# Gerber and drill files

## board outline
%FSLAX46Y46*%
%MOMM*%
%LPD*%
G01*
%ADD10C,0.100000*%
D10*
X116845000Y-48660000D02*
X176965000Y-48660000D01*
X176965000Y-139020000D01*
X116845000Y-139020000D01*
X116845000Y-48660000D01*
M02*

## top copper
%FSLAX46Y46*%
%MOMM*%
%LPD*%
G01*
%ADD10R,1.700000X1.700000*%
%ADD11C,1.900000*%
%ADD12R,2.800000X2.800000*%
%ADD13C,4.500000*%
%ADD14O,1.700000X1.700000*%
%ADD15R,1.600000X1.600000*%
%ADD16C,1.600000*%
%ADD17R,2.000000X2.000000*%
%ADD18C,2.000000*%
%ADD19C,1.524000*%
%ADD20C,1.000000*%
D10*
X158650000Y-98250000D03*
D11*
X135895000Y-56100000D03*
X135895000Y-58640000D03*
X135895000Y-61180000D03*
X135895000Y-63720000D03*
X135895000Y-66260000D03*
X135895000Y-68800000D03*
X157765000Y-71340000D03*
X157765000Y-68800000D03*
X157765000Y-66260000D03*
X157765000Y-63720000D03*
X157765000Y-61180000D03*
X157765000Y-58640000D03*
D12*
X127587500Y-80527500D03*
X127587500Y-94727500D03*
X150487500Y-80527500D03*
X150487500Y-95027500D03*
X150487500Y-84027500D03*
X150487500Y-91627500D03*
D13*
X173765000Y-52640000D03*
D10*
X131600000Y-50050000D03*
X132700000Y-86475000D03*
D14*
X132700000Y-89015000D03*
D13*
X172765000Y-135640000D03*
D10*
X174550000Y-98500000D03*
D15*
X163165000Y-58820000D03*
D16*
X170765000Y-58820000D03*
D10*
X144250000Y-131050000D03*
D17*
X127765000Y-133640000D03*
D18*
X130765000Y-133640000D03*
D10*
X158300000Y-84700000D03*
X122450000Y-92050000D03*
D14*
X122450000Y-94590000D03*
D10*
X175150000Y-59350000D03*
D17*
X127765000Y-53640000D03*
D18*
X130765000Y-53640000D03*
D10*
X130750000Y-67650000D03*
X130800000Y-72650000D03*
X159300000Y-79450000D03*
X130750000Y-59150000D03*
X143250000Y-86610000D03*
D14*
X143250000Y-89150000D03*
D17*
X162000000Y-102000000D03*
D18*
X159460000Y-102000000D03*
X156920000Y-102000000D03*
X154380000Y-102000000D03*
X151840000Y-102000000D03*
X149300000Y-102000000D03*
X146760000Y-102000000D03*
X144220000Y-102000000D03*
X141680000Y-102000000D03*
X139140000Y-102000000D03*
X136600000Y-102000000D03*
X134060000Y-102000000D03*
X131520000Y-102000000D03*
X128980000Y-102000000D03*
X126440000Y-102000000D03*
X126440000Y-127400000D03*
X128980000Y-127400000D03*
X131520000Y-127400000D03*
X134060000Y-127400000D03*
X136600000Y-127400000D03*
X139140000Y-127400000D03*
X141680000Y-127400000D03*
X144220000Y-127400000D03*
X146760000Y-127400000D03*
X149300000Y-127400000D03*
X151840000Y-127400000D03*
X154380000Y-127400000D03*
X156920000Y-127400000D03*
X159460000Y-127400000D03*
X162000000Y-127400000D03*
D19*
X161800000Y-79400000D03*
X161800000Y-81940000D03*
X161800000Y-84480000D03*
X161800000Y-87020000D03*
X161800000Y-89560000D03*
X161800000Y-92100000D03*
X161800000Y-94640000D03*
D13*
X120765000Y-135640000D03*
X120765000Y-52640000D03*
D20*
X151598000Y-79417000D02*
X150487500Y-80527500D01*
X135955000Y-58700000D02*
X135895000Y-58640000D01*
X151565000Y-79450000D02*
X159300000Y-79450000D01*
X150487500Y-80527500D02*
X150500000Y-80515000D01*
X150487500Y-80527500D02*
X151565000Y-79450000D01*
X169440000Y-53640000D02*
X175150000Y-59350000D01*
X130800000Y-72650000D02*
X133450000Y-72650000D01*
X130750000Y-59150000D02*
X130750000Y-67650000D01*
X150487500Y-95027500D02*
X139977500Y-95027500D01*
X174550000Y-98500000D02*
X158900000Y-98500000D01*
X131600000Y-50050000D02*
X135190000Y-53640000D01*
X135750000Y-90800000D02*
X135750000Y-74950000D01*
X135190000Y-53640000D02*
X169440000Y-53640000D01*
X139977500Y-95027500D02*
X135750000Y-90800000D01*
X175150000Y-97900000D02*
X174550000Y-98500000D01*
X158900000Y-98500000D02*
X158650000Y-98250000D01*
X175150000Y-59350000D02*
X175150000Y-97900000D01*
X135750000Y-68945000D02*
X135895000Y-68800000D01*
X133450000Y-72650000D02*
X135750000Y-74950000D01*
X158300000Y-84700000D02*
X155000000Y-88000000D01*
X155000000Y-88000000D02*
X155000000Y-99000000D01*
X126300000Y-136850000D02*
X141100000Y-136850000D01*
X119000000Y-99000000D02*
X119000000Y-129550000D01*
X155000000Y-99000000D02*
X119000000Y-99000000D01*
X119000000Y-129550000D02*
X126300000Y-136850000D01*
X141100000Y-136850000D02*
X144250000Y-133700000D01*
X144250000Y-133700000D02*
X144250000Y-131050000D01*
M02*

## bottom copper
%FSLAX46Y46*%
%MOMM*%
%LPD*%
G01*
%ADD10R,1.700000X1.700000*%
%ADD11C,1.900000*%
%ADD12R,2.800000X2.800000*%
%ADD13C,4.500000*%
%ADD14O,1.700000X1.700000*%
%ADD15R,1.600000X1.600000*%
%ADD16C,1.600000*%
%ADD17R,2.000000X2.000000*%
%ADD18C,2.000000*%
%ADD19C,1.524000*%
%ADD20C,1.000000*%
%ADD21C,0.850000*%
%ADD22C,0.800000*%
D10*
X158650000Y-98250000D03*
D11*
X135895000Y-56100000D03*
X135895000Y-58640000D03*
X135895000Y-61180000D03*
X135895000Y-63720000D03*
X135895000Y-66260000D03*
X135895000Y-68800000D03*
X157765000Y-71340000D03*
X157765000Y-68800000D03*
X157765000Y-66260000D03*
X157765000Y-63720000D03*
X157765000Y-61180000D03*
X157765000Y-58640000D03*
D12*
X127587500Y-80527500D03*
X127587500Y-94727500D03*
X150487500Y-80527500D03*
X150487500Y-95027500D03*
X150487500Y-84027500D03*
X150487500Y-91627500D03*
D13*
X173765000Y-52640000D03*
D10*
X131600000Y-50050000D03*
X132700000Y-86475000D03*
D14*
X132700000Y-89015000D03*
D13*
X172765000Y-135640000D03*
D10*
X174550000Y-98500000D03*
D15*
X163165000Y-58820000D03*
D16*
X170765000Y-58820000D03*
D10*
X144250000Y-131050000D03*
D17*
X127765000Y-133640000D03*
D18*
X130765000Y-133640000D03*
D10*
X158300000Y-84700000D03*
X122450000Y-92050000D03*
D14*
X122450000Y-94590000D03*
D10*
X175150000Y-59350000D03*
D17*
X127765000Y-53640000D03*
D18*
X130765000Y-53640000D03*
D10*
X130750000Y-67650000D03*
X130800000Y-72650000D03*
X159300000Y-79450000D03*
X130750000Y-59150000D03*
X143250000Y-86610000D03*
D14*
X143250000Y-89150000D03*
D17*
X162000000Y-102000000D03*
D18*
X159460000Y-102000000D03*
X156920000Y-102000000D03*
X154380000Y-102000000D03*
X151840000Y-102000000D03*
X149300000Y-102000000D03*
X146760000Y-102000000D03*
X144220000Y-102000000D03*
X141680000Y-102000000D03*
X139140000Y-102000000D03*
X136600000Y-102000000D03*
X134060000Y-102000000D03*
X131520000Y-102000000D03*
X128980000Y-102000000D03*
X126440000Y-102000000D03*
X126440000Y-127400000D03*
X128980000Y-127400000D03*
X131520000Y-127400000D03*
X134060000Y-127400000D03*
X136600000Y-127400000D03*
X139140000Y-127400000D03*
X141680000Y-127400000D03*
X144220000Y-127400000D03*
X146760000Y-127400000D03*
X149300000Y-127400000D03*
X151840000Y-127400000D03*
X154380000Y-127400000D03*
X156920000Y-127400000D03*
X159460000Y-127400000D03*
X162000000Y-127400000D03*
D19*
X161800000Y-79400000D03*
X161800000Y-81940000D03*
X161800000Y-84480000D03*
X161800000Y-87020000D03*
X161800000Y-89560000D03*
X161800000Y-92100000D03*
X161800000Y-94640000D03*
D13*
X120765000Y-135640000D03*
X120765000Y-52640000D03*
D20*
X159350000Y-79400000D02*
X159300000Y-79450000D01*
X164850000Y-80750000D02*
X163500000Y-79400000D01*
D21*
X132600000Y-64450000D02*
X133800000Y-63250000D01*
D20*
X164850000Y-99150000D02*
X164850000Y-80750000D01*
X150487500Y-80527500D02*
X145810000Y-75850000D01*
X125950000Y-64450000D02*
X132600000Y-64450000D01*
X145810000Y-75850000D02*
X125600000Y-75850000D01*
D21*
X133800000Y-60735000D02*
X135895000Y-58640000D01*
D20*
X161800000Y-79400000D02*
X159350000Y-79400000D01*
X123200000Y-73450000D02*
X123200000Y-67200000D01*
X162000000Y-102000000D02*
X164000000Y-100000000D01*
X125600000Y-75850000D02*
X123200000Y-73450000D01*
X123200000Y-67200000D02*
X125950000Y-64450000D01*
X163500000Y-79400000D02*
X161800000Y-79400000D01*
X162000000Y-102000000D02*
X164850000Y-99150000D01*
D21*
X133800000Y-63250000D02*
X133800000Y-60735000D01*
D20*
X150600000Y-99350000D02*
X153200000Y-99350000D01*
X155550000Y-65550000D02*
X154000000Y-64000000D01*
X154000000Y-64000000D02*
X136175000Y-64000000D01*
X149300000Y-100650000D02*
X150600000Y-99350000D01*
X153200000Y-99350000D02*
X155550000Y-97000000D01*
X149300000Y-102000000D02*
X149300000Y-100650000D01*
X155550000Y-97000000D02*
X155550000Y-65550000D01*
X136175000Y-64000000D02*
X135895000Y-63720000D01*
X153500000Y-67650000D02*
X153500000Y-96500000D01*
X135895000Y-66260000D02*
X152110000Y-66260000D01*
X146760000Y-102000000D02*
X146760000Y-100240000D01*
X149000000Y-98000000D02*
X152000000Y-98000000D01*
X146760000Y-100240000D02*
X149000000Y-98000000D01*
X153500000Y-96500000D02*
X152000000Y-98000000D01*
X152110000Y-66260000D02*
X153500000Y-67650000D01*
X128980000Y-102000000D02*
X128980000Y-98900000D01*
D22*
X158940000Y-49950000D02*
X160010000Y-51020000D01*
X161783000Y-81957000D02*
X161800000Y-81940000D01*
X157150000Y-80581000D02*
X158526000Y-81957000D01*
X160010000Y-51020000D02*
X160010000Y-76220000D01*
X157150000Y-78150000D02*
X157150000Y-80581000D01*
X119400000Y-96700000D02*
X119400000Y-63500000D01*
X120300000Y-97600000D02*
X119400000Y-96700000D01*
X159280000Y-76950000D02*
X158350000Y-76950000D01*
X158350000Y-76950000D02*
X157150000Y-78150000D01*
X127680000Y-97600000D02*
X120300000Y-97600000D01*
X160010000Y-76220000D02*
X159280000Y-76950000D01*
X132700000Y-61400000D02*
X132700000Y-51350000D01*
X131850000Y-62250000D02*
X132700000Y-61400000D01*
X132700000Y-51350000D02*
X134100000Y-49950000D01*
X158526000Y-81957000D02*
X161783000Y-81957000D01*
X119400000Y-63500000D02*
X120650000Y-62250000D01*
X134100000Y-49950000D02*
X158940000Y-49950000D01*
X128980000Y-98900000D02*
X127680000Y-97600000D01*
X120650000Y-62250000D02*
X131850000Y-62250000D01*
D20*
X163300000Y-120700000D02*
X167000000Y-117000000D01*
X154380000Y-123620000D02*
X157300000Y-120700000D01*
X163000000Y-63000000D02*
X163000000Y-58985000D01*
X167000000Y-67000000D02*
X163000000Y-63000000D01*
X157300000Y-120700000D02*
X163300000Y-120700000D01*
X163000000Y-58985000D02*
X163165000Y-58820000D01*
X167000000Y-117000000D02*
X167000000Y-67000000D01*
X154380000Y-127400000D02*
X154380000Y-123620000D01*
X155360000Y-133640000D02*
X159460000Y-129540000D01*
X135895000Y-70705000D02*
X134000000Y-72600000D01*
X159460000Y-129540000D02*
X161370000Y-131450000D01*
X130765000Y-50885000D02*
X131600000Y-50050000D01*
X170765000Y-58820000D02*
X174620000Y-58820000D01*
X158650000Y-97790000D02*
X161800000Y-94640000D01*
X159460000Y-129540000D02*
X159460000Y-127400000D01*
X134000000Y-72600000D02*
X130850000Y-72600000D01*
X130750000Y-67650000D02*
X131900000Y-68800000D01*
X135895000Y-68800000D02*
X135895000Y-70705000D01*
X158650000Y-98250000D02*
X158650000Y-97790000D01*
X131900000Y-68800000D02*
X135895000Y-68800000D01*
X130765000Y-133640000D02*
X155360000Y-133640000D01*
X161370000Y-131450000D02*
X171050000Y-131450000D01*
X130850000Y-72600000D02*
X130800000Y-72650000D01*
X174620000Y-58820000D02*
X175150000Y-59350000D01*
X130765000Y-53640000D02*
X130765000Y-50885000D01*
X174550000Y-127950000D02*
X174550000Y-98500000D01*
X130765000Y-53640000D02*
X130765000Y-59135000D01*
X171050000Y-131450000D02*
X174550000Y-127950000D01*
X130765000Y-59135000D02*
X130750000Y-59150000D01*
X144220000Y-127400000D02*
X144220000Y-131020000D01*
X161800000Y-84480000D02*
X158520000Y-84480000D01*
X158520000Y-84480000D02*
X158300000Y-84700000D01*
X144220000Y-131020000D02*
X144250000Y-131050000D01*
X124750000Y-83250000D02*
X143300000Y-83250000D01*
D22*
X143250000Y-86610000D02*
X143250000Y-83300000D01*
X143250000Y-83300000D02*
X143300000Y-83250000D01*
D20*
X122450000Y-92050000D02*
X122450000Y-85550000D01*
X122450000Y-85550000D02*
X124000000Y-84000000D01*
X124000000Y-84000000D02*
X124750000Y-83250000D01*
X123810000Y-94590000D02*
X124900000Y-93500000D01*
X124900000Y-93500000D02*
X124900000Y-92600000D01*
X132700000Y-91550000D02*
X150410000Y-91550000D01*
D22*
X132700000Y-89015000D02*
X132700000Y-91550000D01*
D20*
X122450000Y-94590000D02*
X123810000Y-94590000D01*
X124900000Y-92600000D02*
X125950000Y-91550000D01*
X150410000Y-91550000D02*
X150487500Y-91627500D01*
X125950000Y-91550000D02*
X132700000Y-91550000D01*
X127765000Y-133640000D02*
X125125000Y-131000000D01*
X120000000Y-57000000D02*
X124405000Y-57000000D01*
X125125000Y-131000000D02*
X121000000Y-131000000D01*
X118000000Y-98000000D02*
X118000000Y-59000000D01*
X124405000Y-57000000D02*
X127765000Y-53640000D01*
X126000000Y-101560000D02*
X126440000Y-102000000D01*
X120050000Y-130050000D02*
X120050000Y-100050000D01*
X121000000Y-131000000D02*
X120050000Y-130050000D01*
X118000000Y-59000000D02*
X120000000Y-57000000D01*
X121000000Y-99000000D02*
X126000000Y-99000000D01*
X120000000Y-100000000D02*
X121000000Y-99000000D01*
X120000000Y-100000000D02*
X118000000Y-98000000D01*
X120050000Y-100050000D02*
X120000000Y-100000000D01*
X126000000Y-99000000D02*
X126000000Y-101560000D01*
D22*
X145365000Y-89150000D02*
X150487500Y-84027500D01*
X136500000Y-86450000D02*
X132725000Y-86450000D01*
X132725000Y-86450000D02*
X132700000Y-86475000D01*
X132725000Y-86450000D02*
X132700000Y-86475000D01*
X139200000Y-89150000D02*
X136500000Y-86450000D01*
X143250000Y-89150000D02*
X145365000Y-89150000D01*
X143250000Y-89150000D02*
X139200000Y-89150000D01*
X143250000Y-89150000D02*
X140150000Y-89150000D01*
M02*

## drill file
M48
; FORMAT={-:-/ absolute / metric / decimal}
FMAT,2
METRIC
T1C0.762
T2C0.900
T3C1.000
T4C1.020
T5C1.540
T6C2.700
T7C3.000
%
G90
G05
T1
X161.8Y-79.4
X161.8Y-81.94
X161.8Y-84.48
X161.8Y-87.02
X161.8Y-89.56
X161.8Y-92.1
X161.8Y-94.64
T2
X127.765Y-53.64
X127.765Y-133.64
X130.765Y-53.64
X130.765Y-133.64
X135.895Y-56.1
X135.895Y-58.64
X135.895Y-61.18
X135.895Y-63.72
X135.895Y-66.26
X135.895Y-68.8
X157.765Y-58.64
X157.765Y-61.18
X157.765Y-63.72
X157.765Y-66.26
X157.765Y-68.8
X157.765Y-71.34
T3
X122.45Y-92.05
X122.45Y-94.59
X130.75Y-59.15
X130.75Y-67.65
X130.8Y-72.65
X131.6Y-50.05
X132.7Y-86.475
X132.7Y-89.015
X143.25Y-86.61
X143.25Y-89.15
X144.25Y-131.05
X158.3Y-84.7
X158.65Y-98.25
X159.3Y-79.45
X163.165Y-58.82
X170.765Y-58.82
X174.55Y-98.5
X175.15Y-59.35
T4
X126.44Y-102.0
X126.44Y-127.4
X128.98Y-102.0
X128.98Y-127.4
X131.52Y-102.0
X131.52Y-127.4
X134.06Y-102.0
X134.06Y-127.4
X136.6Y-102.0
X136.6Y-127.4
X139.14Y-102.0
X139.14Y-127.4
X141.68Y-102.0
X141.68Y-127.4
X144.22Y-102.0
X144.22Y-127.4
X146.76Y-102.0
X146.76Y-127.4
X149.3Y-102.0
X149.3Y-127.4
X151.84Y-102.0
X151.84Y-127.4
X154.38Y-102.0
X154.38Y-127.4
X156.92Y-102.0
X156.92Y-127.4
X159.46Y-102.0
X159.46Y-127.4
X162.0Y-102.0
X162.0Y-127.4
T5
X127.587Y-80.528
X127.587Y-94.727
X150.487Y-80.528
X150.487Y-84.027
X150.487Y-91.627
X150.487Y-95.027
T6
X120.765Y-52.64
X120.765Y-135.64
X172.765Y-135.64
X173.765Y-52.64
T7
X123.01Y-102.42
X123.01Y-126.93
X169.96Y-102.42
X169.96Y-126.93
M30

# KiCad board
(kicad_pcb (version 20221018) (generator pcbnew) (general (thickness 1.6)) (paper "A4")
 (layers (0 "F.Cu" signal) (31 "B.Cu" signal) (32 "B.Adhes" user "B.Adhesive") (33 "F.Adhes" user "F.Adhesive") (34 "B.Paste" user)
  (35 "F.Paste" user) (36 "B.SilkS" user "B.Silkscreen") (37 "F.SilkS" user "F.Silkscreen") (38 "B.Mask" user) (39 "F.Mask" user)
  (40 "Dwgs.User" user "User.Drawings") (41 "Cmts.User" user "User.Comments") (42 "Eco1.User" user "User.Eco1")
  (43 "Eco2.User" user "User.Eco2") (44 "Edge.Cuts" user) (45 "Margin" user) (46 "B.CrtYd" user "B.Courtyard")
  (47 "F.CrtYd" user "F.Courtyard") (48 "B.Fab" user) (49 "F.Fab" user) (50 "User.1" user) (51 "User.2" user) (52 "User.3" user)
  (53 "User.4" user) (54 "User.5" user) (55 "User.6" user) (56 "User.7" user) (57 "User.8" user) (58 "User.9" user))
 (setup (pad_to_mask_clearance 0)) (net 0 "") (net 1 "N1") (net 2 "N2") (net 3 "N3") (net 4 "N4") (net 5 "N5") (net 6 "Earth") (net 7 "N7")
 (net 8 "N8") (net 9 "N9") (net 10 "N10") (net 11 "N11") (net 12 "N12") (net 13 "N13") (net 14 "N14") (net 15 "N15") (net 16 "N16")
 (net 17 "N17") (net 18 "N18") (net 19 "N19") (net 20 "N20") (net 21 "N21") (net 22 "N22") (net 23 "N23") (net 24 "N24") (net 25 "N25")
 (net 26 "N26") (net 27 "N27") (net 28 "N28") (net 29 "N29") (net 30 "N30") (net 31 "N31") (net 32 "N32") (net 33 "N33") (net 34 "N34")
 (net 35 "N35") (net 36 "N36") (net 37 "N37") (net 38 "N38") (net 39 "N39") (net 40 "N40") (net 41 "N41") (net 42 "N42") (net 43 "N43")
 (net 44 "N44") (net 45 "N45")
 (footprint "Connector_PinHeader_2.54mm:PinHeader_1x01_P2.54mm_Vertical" (layer "F.Cu") (at 158.65 98.25)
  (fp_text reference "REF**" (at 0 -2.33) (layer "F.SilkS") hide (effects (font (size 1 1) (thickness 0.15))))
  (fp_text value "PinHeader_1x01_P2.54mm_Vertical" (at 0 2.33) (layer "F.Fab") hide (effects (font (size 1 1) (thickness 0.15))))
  (pad "1" thru_hole rect (at 0 0) (size 1.7 1.7) (drill 1) (layers "*.Cu" "*.Mask")))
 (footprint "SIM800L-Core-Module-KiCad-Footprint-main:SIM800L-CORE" (layer "F.Cu") (at 135.895 56.1)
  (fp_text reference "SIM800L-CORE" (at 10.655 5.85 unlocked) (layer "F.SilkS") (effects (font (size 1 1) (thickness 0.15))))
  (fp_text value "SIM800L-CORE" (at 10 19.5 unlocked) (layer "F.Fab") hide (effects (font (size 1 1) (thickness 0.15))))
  (pad "1" thru_hole circle (at 0 0) (size 1.9 1.9) (drill 0.9) (layers "*.Cu" "*.Mask") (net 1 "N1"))
  (pad "2" thru_hole circle (at 0 2.54) (size 1.9 1.9) (drill 0.9) (layers "*.Cu" "*.Mask") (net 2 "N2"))
  (pad "3" thru_hole circle (at 0 5.08) (size 1.9 1.9) (drill 0.9) (layers "*.Cu" "*.Mask") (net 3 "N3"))
  (pad "4" thru_hole circle (at 0 7.62) (size 1.9 1.9) (drill 0.9) (layers "*.Cu" "*.Mask") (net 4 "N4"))
  (pad "5" thru_hole circle (at 0 10.16) (size 1.9 1.9) (drill 0.9) (layers "*.Cu" "*.Mask") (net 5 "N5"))
  (pad "6" thru_hole circle (at 0 12.7) (size 1.9 1.9) (drill 0.9) (layers "*.Cu" "*.Mask") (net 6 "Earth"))
  (pad "7" thru_hole circle (at 21.87 15.24) (size 1.9 1.9) (drill 0.9) (layers "*.Cu" "*.Mask") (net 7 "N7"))
  (pad "8" thru_hole circle (at 21.87 12.7) (size 1.9 1.9) (drill 0.9) (layers "*.Cu" "*.Mask") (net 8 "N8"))
  (pad "9" thru_hole circle (at 21.87 10.16) (size 1.9 1.9) (drill 0.9) (layers "*.Cu" "*.Mask") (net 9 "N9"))
  (pad "10" thru_hole circle (at 21.87 7.62) (size 1.9 1.9) (drill 0.9) (layers "*.Cu" "*.Mask") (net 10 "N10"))
  (pad "11" thru_hole circle (at 21.87 5.08) (size 1.9 1.9) (drill 0.9) (layers "*.Cu" "*.Mask") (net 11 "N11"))
  (pad "12" thru_hole circle (at 21.87 2.54) (size 1.9 1.9) (drill 0.9) (layers "*.Cu" "*.Mask") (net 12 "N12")))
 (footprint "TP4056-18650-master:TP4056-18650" (layer "F.Cu") (at 125.8875 78.8275)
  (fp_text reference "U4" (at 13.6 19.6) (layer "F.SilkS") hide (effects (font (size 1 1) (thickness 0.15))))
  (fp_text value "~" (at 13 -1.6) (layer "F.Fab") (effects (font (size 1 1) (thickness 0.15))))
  (pad "1" thru_hole rect (at 1.7 1.7) (size 2.8 2.8) (drill 1.54) (layers "*.Cu" "*.Mask") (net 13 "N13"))
  (pad "2" thru_hole rect (at 1.7 15.9) (size 2.8 2.8) (drill 1.54) (layers "*.Cu" "*.Mask") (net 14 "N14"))
  (pad "3" thru_hole rect (at 24.6 1.7) (size 2.8 2.8) (drill 1.54) (layers "*.Cu" "*.Mask") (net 2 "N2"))
  (pad "4" thru_hole rect (at 24.6 16.2) (size 2.8 2.8) (drill 1.54) (layers "*.Cu" "*.Mask") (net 6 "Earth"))
  (pad "5" thru_hole rect (at 24.6 5.2) (size 2.8 2.8) (drill 1.54) (layers "*.Cu" "*.Mask") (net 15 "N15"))
  (pad "6" thru_hole rect (at 24.6 12.8) (size 2.8 2.8) (drill 1.54) (layers "*.Cu" "*.Mask") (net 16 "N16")))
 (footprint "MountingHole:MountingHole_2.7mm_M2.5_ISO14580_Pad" (layer "F.Cu") (at 173.765 52.64)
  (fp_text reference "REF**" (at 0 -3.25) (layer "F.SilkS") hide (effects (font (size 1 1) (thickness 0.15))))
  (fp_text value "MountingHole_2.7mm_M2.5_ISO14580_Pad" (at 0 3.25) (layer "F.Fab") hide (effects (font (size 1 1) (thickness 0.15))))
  (pad "1" thru_hole circle (at 0 0) (size 4.5 4.5) (drill 2.7) (layers "*.Cu" "*.Mask")))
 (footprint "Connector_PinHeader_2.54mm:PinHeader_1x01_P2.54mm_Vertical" (layer "F.Cu") (at 131.6 50.05)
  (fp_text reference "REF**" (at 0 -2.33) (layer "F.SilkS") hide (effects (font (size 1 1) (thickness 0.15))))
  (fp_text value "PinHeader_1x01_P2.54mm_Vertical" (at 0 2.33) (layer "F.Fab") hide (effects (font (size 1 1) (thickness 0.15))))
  (pad "1" thru_hole rect (at 0 0) (size 1.7 1.7) (drill 1) (layers "*.Cu" "*.Mask")))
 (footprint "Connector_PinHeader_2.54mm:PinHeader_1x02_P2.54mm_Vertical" (layer "F.Cu") (at 132.7 86.475)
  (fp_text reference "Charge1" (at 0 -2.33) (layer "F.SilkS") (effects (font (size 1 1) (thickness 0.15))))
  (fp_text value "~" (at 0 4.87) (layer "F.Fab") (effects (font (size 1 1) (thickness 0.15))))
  (pad "1" thru_hole rect (at 0 0) (size 1.7 1.7) (drill 1) (layers "*.Cu" "*.Mask") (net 15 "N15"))
  (pad "2" thru_hole oval (at 0 2.54) (size 1.7 1.7) (drill 1) (layers "*.Cu" "*.Mask") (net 16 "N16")))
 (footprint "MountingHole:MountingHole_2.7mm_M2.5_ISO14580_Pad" (layer "F.Cu") (at 172.765 135.64)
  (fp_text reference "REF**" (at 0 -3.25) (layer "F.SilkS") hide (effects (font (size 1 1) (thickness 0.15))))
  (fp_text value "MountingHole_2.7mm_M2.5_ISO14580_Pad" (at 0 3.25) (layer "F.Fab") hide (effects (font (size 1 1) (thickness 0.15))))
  (pad "1" thru_hole circle (at 0 0) (size 4.5 4.5) (drill 2.7) (layers "*.Cu" "*.Mask")))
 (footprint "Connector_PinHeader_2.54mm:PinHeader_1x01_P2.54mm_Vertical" (layer "F.Cu") (at 174.55 98.5)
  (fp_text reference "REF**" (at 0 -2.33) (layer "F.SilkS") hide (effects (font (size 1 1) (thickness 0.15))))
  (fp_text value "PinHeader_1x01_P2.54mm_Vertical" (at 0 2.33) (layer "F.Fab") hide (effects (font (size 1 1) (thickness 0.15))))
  (pad "1" thru_hole rect (at 0 0) (size 1.7 1.7) (drill 1) (layers "*.Cu" "*.Mask")))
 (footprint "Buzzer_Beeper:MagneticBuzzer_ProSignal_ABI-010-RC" (layer "F.Cu") (at 163.165 58.82)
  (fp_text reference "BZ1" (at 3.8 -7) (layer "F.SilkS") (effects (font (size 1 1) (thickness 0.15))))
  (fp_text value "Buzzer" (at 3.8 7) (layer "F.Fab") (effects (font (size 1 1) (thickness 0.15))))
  (pad "1" thru_hole rect (at 0 0) (size 1.6 1.6) (drill 1) (layers "*.Cu" "*.Mask") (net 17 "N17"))
  (pad "2" thru_hole circle (at 7.6 0) (size 1.6 1.6) (drill 1) (layers "*.Cu" "*.Mask") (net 6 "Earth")))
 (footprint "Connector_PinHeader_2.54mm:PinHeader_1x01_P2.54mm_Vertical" (layer "F.Cu") (at 144.25 131.05)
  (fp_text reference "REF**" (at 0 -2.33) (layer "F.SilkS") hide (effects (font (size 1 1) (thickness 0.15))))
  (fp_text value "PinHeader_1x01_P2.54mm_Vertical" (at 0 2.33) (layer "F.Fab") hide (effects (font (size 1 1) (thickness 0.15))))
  (pad "1" thru_hole rect (at 0 0) (size 1.7 1.7) (drill 1) (layers "*.Cu" "*.Mask")))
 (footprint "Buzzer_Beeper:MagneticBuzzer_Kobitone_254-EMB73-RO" (layer "F.Cu") (at 127.765 133.64)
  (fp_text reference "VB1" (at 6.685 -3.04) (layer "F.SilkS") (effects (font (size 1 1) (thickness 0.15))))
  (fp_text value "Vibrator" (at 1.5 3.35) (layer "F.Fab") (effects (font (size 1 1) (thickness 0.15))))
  (pad "1" thru_hole rect (at 0 0) (size 2 2) (drill 0.9) (layers "*.Cu" "*.Mask") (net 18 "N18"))
  (pad "2" thru_hole circle (at 3 0) (size 2 2) (drill 0.9) (layers "*.Cu" "*.Mask") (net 6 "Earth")))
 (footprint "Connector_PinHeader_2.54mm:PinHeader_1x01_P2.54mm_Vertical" (layer "F.Cu") (at 158.3 84.7)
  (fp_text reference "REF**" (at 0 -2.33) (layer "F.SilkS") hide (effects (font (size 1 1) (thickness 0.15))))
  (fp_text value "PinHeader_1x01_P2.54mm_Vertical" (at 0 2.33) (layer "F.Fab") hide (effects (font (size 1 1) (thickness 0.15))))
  (pad "1" thru_hole rect (at 0 0) (size 1.7 1.7) (drill 1) (layers "*.Cu" "*.Mask")))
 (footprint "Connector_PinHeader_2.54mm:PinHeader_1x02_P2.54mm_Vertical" (layer "F.Cu") (at 122.45 92.05)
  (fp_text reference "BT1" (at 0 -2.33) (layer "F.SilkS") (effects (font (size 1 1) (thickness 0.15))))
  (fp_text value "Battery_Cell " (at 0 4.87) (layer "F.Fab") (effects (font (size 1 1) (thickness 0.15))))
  (pad "1" thru_hole rect (at 0 0) (size 1.7 1.7) (drill 1) (layers "*.Cu" "*.Mask") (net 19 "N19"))
  (pad "2" thru_hole oval (at 0 2.54) (size 1.7 1.7) (drill 1) (layers "*.Cu" "*.Mask") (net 16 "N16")))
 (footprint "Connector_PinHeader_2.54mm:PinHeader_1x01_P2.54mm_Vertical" (layer "F.Cu") (at 175.15 59.35)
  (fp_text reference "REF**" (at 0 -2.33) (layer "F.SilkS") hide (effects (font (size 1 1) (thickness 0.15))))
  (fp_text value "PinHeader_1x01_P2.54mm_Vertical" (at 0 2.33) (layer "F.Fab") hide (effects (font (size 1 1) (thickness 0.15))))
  (pad "1" thru_hole rect (at 0 0) (size 1.7 1.7) (drill 1) (layers "*.Cu" "*.Mask")))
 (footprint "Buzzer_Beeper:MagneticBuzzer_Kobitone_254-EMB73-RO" (layer "F.Cu") (at 127.765 53.64)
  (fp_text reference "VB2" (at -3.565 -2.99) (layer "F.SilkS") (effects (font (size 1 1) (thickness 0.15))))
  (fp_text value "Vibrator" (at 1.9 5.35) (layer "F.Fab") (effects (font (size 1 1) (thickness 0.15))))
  (pad "1" thru_hole rect (at 0 0) (size 2 2) (drill 0.9) (layers "*.Cu" "*.Mask") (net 18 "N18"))
  (pad "2" thru_hole circle (at 3 0) (size 2 2) (drill 0.9) (layers "*.Cu" "*.Mask") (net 6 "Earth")))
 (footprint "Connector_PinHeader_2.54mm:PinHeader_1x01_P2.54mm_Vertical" (layer "F.Cu") (at 130.75 67.65)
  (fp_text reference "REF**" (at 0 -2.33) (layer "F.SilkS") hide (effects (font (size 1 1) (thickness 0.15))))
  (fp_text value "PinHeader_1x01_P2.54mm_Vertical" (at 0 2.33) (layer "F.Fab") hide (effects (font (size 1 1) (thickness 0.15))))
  (pad "1" thru_hole rect (at 0 0) (size 1.7 1.7) (drill 1) (layers "*.Cu" "*.Mask")))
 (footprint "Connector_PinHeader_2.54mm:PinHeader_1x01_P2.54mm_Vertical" (layer "F.Cu") (at 130.8 72.65)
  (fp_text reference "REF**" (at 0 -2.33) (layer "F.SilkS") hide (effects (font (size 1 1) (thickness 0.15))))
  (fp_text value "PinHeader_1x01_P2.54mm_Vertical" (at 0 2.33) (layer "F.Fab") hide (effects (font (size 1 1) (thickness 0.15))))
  (pad "1" thru_hole rect (at 0 0) (size 1.7 1.7) (drill 1) (layers "*.Cu" "*.Mask")))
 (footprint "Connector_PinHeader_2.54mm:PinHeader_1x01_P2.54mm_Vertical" (layer "F.Cu") (at 159.3 79.45)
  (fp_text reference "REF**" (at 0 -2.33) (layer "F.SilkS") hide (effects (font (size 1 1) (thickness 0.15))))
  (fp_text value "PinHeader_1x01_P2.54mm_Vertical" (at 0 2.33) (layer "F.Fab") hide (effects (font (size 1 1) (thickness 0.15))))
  (pad "1" thru_hole rect (at 0 0) (size 1.7 1.7) (drill 1) (layers "*.Cu" "*.Mask") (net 2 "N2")))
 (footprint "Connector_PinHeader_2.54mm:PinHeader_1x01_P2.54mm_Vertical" (layer "F.Cu") (at 130.75 59.15)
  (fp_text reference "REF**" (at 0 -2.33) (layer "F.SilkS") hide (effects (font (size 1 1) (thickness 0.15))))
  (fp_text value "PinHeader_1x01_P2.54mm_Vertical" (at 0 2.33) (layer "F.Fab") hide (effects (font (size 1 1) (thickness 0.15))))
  (pad "1" thru_hole rect (at 0 0) (size 1.7 1.7) (drill 1) (layers "*.Cu" "*.Mask")))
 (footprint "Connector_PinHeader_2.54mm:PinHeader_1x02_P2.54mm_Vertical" (layer "F.Cu") (at 143.25 86.61)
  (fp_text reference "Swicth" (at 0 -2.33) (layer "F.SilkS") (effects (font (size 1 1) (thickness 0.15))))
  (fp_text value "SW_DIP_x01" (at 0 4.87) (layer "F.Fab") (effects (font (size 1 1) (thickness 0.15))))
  (pad "1" thru_hole rect (at 0 0) (size 1.7 1.7) (drill 1) (layers "*.Cu" "*.Mask") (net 19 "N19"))
  (pad "2" thru_hole oval (at 0 2.54) (size 1.7 1.7) (drill 1) (layers "*.Cu" "*.Mask") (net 15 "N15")))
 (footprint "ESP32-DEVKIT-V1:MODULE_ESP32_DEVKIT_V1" (layer "F.Cu") (at 146.485 114.7 -90)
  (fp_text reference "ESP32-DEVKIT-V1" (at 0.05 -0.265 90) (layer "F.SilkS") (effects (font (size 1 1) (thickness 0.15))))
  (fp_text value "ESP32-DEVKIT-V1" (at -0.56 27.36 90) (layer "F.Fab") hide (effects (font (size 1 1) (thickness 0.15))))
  (pad "" np_thru_hole circle (at -12.28 -23.475 270) (size 3 3) (drill 3) (layers "*.Cu" "*.Mask"))
  (pad "" np_thru_hole circle (at -12.28 23.475 270) (size 3 3) (drill 3) (layers "*.Cu" "*.Mask"))
  (pad "" np_thru_hole circle (at 12.23 -23.475 270) (size 3 3) (drill 3) (layers "*.Cu" "*.Mask"))
  (pad "" np_thru_hole circle (at 12.23 23.475 270) (size 3 3) (drill 3) (layers "*.Cu" "*.Mask"))
  (pad "1" thru_hole rect (at -12.7 -15.515 270) (size 2 2) (drill 1.02) (layers "*.Cu" "*.Mask") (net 2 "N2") (solder_mask_margin 0.102))
  (pad "2" thru_hole circle (at -12.7 -12.975 270) (size 2 2) (drill 1.02) (layers "*.Cu" "*.Mask") (solder_mask_margin 0.102))
  (pad "3" thru_hole circle (at -12.7 -10.435 270) (size 2 2) (drill 1.02) (layers "*.Cu" "*.Mask") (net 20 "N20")
   (solder_mask_margin 0.102))
  (pad "4" thru_hole circle (at -12.7 -7.895 270) (size 2 2) (drill 1.02) (layers "*.Cu" "*.Mask") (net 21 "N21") (solder_mask_margin 0.102))
  (pad "5" thru_hole circle (at -12.7 -5.355 270) (size 2 2) (drill 1.02) (layers "*.Cu" "*.Mask") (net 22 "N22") (solder_mask_margin 0.102))
  (pad "6" thru_hole circle (at -12.7 -2.815 270) (size 2 2) (drill 1.02) (layers "*.Cu" "*.Mask") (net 4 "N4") (solder_mask_margin 0.102))
  (pad "7" thru_hole circle (at -12.7 -0.275 270) (size 2 2) (drill 1.02) (layers "*.Cu" "*.Mask") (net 5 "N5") (solder_mask_margin 0.102))
  (pad "8" thru_hole circle (at -12.7 2.265 270) (size 2 2) (drill 1.02) (layers "*.Cu" "*.Mask") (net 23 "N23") (solder_mask_margin 0.102))
  (pad "9" thru_hole circle (at -12.7 4.805 270) (size 2 2) (drill 1.02) (layers "*.Cu" "*.Mask") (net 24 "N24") (solder_mask_margin 0.102))
  (pad "10" thru_hole circle (at -12.7 7.345 270) (size 2 2) (drill 1.02) (layers "*.Cu" "*.Mask") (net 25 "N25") (solder_mask_margin 0.102))
  (pad "11" thru_hole circle (at -12.7 9.885 270) (size 2 2) (drill 1.02) (layers "*.Cu" "*.Mask") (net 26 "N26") (solder_mask_margin 0.102))
  (pad "12" thru_hole circle (at -12.7 12.425 270) (size 2 2) (drill 1.02) (layers "*.Cu" "*.Mask") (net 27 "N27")
   (solder_mask_margin 0.102))
  (pad "13" thru_hole circle (at -12.7 14.965 270) (size 2 2) (drill 1.02) (layers "*.Cu" "*.Mask") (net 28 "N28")
   (solder_mask_margin 0.102))
  (pad "14" thru_hole circle (at -12.7 17.505 270) (size 2 2) (drill 1.02) (layers "*.Cu" "*.Mask") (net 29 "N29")
   (solder_mask_margin 0.102))
  (pad "15" thru_hole circle (at -12.7 20.045 270) (size 2 2) (drill 1.02) (layers "*.Cu" "*.Mask") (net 18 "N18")
   (solder_mask_margin 0.102))
  (pad "16" thru_hole circle (at 12.7 20.045 270) (size 2 2) (drill 1.02) (layers "*.Cu" "*.Mask") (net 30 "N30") (solder_mask_margin 0.102))
  (pad "17" thru_hole circle (at 12.7 17.505 270) (size 2 2) (drill 1.02) (layers "*.Cu" "*.Mask") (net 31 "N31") (solder_mask_margin 0.102))
  (pad "18" thru_hole circle (at 12.7 14.965 270) (size 2 2) (drill 1.02) (layers "*.Cu" "*.Mask") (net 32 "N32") (solder_mask_margin 0.102))
  (pad "19" thru_hole circle (at 12.7 12.425 270) (size 2 2) (drill 1.02) (layers "*.Cu" "*.Mask") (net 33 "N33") (solder_mask_margin 0.102))
  (pad "20" thru_hole circle (at 12.7 9.885 270) (size 2 2) (drill 1.02) (layers "*.Cu" "*.Mask") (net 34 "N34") (solder_mask_margin 0.102))
  (pad "21" thru_hole circle (at 12.7 7.345 270) (size 2 2) (drill 1.02) (layers "*.Cu" "*.Mask") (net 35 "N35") (solder_mask_margin 0.102))
  (pad "22" thru_hole circle (at 12.7 4.805 270) (size 2 2) (drill 1.02) (layers "*.Cu" "*.Mask") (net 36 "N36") (solder_mask_margin 0.102))
  (pad "23" thru_hole circle (at 12.7 2.265 270) (size 2 2) (drill 1.02) (layers "*.Cu" "*.Mask") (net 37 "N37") (solder_mask_margin 0.102))
  (pad "24" thru_hole circle (at 12.7 -0.275 270) (size 2 2) (drill 1.02) (layers "*.Cu" "*.Mask") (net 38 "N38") (solder_mask_margin 0.102))
  (pad "25" thru_hole circle (at 12.7 -2.815 270) (size 2 2) (drill 1.02) (layers "*.Cu" "*.Mask") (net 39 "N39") (solder_mask_margin 0.102))
  (pad "26" thru_hole circle (at 12.7 -5.355 270) (size 2 2) (drill 1.02) (layers "*.Cu" "*.Mask") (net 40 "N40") (solder_mask_margin 0.102))
  (pad "27" thru_hole circle (at 12.7 -7.895 270) (size 2 2) (drill 1.02) (layers "*.Cu" "*.Mask") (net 17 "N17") (solder_mask_margin 0.102))
  (pad "28" thru_hole circle (at 12.7 -10.435 270) (size 2 2) (drill 1.02) (layers "*.Cu" "*.Mask") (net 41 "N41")
   (solder_mask_margin 0.102))
  (pad "29" thru_hole circle (at 12.7 -12.975 270) (size 2 2) (drill 1.02) (layers "*.Cu" "*.Mask") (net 6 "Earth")
   (solder_mask_margin 0.102))
  (pad "30" thru_hole circle (at 12.7 -15.515 270) (size 2 2) (drill 1.02) (layers "*.Cu" "*.Mask") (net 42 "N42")
   (solder_mask_margin 0.102))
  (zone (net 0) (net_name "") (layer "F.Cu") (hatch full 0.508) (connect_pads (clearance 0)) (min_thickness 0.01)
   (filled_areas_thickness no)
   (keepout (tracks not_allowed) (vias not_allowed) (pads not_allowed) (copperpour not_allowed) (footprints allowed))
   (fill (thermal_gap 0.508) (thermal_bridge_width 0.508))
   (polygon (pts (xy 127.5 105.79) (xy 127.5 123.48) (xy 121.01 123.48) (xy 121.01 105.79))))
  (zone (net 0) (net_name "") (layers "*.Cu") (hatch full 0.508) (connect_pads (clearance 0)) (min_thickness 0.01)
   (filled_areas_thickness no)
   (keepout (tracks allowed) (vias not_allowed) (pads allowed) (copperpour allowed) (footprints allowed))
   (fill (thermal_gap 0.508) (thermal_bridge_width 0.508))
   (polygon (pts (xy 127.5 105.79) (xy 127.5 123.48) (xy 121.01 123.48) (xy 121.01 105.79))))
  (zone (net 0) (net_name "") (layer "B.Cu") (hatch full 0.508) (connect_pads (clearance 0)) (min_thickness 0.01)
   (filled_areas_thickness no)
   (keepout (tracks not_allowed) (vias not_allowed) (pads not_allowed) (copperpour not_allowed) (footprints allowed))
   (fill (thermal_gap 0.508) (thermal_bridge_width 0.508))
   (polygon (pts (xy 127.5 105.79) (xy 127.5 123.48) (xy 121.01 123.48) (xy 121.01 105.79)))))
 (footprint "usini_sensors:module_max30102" (layer "F.Cu") (at 159.26 97.18)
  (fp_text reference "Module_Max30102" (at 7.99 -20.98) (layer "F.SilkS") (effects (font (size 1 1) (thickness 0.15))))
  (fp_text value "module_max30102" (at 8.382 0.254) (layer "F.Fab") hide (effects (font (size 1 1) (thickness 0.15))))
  (pad "1" thru_hole circle (at 2.54 -17.78) (size 1.524 1.524) (drill 0.762) (layers "*.Cu" "*.Mask") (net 2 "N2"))
  (pad "2" thru_hole circle (at 2.54 -15.24) (size 1.524 1.524) (drill 0.762) (layers "*.Cu" "*.Mask") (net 29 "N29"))
  (pad "3" thru_hole circle (at 2.54 -12.7) (size 1.524 1.524) (drill 0.762) (layers "*.Cu" "*.Mask") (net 37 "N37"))
  (pad "4" thru_hole circle (at 2.54 -10.16) (size 1.524 1.524) (drill 0.762) (layers "*.Cu" "*.Mask") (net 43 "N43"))
  (pad "5" thru_hole circle (at 2.54 -7.62) (size 1.524 1.524) (drill 0.762) (layers "*.Cu" "*.Mask") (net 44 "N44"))
  (pad "6" thru_hole circle (at 2.54 -5.08) (size 1.524 1.524) (drill 0.762) (layers "*.Cu" "*.Mask") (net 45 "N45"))
  (pad "7" thru_hole circle (at 2.54 -2.54) (size 1.524 1.524) (drill 0.762) (layers "*.Cu" "*.Mask") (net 6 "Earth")))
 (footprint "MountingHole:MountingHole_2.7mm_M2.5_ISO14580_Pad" (layer "F.Cu") (at 120.765 135.64)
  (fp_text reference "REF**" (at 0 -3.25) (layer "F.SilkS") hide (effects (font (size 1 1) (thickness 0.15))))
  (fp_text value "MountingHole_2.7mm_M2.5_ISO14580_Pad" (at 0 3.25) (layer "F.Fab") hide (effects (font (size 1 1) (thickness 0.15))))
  (pad "1" thru_hole circle (at 0 0) (size 4.5 4.5) (drill 2.7) (layers "*.Cu" "*.Mask")))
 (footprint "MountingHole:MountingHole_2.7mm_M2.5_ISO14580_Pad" (layer "F.Cu") (at 120.765 52.64)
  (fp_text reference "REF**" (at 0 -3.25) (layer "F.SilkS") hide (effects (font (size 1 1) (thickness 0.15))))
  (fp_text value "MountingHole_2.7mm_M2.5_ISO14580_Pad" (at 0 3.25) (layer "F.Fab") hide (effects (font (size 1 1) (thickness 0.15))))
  (pad "1" thru_hole circle (at 0 0) (size 4.5 4.5) (drill 2.7) (layers "*.Cu" "*.Mask")))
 (gr_rect locked (start 116.845 48.66) (end 176.965 139.02) (stroke (width 0.1) (type default)) (fill none) (layer "Edge.Cuts"))
 (segment (start 151.598 79.417) (end 150.4875 80.5275) (width 1) (layer "F.Cu") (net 2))
 (segment (start 135.955 58.7) (end 135.895 58.64) (width 1) (layer "F.Cu") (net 2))
 (segment (start 151.565 79.45) (end 159.3 79.45) (width 1) (layer "F.Cu") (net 2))
 (segment (start 150.4875 80.5275) (end 150.5 80.515) (width 1) (layer "F.Cu") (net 2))
 (segment (start 150.4875 80.5275) (end 151.565 79.45) (width 1) (layer "F.Cu") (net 2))
 (segment (start 159.35 79.4) (end 159.3 79.45) (width 1) (layer "B.Cu") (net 2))
 (segment (start 164.85 80.75) (end 163.5 79.4) (width 1) (layer "B.Cu") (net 2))
 (segment (start 132.6 64.45) (end 133.8 63.25) (width 0.85) (layer "B.Cu") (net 2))
 (segment (start 164.85 99.15) (end 164.85 80.75) (width 1) (layer "B.Cu") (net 2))
 (segment (start 150.4875 80.5275) (end 145.81 75.85) (width 1) (layer "B.Cu") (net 2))
 (segment (start 125.95 64.45) (end 132.6 64.45) (width 1) (layer "B.Cu") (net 2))
 (segment (start 145.81 75.85) (end 125.6 75.85) (width 1) (layer "B.Cu") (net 2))
 (segment (start 133.8 60.735) (end 135.895 58.64) (width 0.85) (layer "B.Cu") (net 2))
 (segment (start 161.8 79.4) (end 159.35 79.4) (width 1) (layer "B.Cu") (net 2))
 (segment (start 123.2 73.45) (end 123.2 67.2) (width 1) (layer "B.Cu") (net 2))
 (segment (start 162 102) (end 164 100) (width 1) (layer "B.Cu") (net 2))
 (segment (start 125.6 75.85) (end 123.2 73.45) (width 1) (layer "B.Cu") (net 2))
 (segment (start 123.2 67.2) (end 125.95 64.45) (width 1) (layer "B.Cu") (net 2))
 (segment (start 163.5 79.4) (end 161.8 79.4) (width 1) (layer "B.Cu") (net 2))
 (segment (start 162 102) (end 164.85 99.15) (width 1) (layer "B.Cu") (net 2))
 (segment (start 133.8 63.25) (end 133.8 60.735) (width 0.85) (layer "B.Cu") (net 2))
 (segment (start 150.6 99.35) (end 153.2 99.35) (width 1) (layer "B.Cu") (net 4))
 (segment (start 155.55 65.55) (end 154 64) (width 1) (layer "B.Cu") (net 4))
 (segment (start 154 64) (end 136.175 64) (width 1) (layer "B.Cu") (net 4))
 (segment (start 149.3 100.65) (end 150.6 99.35) (width 1) (layer "B.Cu") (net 4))
 (segment (start 153.2 99.35) (end 155.55 97) (width 1) (layer "B.Cu") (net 4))
 (segment (start 149.3 102) (end 149.3 100.65) (width 1) (layer "B.Cu") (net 4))
 (segment (start 155.55 97) (end 155.55 65.55) (width 1) (layer "B.Cu") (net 4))
 (segment (start 136.175 64) (end 135.895 63.72) (width 1) (layer "B.Cu") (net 4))
 (segment (start 153.5 67.65) (end 153.5 96.5) (width 1) (layer "B.Cu") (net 5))
 (segment (start 135.895 66.26) (end 152.11 66.26) (width 1) (layer "B.Cu") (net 5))
 (segment (start 146.76 102) (end 146.76 100.24) (width 1) (layer "B.Cu") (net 5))
 (segment (start 149 98) (end 152 98) (width 1) (layer "B.Cu") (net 5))
 (segment (start 146.76 100.24) (end 149 98) (width 1) (layer "B.Cu") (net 5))
 (segment (start 153.5 96.5) (end 152 98) (width 1) (layer "B.Cu") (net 5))
 (segment (start 152.11 66.26) (end 153.5 67.65) (width 1) (layer "B.Cu") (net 5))
 (segment (start 128.98 102) (end 128.98 98.9) (width 1) (layer "B.Cu") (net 29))
 (segment (start 158.94 49.95) (end 160.01 51.02) (width 0.8) (layer "B.Cu") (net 29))
 (segment (start 161.783 81.957) (end 161.8 81.94) (width 0.8) (layer "B.Cu") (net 29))
 (segment (start 157.15 80.581) (end 158.526 81.957) (width 0.8) (layer "B.Cu") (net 29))
 (segment (start 160.01 51.02) (end 160.01 76.22) (width 0.8) (layer "B.Cu") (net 29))
 (segment (start 157.15 78.15) (end 157.15 80.581) (width 0.8) (layer "B.Cu") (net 29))
 (segment (start 119.4 96.7) (end 119.4 63.5) (width 0.8) (layer "B.Cu") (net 29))
 (segment (start 120.3 97.6) (end 119.4 96.7) (width 0.8) (layer "B.Cu") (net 29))
 (segment (start 159.28 76.95) (end 158.35 76.95) (width 0.8) (layer "B.Cu") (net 29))
 (segment (start 158.35 76.95) (end 157.15 78.15) (width 0.8) (layer "B.Cu") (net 29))
 (segment (start 127.68 97.6) (end 120.3 97.6) (width 0.8) (layer "B.Cu") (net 29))
 (segment (start 160.01 76.22) (end 159.28 76.95) (width 0.8) (layer "B.Cu") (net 29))
 (segment (start 132.7 61.4) (end 132.7 51.35) (width 0.8) (layer "B.Cu") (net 29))
 (segment (start 131.85 62.25) (end 132.7 61.4) (width 0.8) (layer "B.Cu") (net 29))
 (segment (start 132.7 51.35) (end 134.1 49.95) (width 0.8) (layer "B.Cu") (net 29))
 (segment (start 158.526 81.957) (end 161.783 81.957) (width 0.8) (layer "B.Cu") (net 29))
 (segment (start 119.4 63.5) (end 120.65 62.25) (width 0.8) (layer "B.Cu") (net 29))
 (segment (start 134.1 49.95) (end 158.94 49.95) (width 0.8) (layer "B.Cu") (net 29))
 (segment (start 128.98 98.9) (end 127.68 97.6) (width 0.8) (layer "B.Cu") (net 29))
 (segment (start 120.65 62.25) (end 131.85 62.25) (width 0.8) (layer "B.Cu") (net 29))
 (segment (start 163.3 120.7) (end 167 117) (width 1) (layer "B.Cu") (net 17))
 (segment (start 154.38 123.62) (end 157.3 120.7) (width 1) (layer "B.Cu") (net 17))
 (segment (start 163 63) (end 163 58.985) (width 1) (layer "B.Cu") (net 17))
 (segment (start 167 67) (end 163 63) (width 1) (layer "B.Cu") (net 17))
 (segment (start 157.3 120.7) (end 163.3 120.7) (width 1) (layer "B.Cu") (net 17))
 (segment (start 163 58.985) (end 163.165 58.82) (width 1) (layer "B.Cu") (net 17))
 (segment (start 167 117) (end 167 67) (width 1) (layer "B.Cu") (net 17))
 (segment (start 154.38 127.4) (end 154.38 123.62) (width 1) (layer "B.Cu") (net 17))
 (segment (start 169.44 53.64) (end 175.15 59.35) (width 1) (layer "F.Cu") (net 6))
 (segment (start 130.8 72.65) (end 133.45 72.65) (width 1) (layer "F.Cu") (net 6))
 (segment (start 130.75 59.15) (end 130.75 67.65) (width 1) (layer "F.Cu") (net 6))
 (segment (start 150.4875 95.0275) (end 139.9775 95.0275) (width 1) (layer "F.Cu") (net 6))
 (segment (start 174.55 98.5) (end 158.9 98.5) (width 1) (layer "F.Cu") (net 6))
 (segment (start 131.6 50.05) (end 135.19 53.64) (width 1) (layer "F.Cu") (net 6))
 (segment (start 135.75 90.8) (end 135.75 74.95) (width 1) (layer "F.Cu") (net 6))
 (segment (start 135.19 53.64) (end 169.44 53.64) (width 1) (layer "F.Cu") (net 6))
 (segment (start 139.9775 95.0275) (end 135.75 90.8) (width 1) (layer "F.Cu") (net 6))
 (segment (start 175.15 97.9) (end 174.55 98.5) (width 1) (layer "F.Cu") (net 6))
 (segment (start 158.9 98.5) (end 158.65 98.25) (width 1) (layer "F.Cu") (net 6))
 (segment (start 175.15 59.35) (end 175.15 97.9) (width 1) (layer "F.Cu") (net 6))
 (segment (start 135.75 68.945) (end 135.895 68.8) (width 1) (layer "F.Cu") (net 6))
 (segment (start 133.45 72.65) (end 135.75 74.95) (width 1) (layer "F.Cu") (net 6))
 (segment (start 155.36 133.64) (end 159.46 129.54) (width 1) (layer "B.Cu") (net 6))
 (segment (start 135.895 70.705) (end 134 72.6) (width 1) (layer "B.Cu") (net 6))
 (segment (start 159.46 129.54) (end 161.37 131.45) (width 1) (layer "B.Cu") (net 6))
 (segment (start 130.765 50.885) (end 131.6 50.05) (width 1) (layer "B.Cu") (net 6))
 (segment (start 170.765 58.82) (end 174.62 58.82) (width 1) (layer "B.Cu") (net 6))
 (segment (start 158.65 97.79) (end 161.8 94.64) (width 1) (layer "B.Cu") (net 6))
 (segment (start 159.46 129.54) (end 159.46 127.4) (width 1) (layer "B.Cu") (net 6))
 (segment (start 134 72.6) (end 130.85 72.6) (width 1) (layer "B.Cu") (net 6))
 (segment (start 130.75 67.65) (end 131.9 68.8) (width 1) (layer "B.Cu") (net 6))
 (segment (start 135.895 68.8) (end 135.895 70.705) (width 1) (layer "B.Cu") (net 6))
 (segment (start 158.65 98.25) (end 158.65 97.79) (width 1) (layer "B.Cu") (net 6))
 (segment (start 131.9 68.8) (end 135.895 68.8) (width 1) (layer "B.Cu") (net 6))
 (segment (start 130.765 133.64) (end 155.36 133.64) (width 1) (layer "B.Cu") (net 6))
 (segment (start 161.37 131.45) (end 171.05 131.45) (width 1) (layer "B.Cu") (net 6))
 (segment (start 130.85 72.6) (end 130.8 72.65) (width 1) (layer "B.Cu") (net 6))
 (segment (start 174.62 58.82) (end 175.15 59.35) (width 1) (layer "B.Cu") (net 6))
 (segment (start 130.765 53.64) (end 130.765 50.885) (width 1) (layer "B.Cu") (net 6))
 (segment (start 174.55 127.95) (end 174.55 98.5) (width 1) (layer "B.Cu") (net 6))
 (segment (start 130.765 53.64) (end 130.765 59.135) (width 1) (layer "B.Cu") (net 6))
 (segment (start 171.05 131.45) (end 174.55 127.95) (width 1) (layer "B.Cu") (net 6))
 (segment (start 130.765 59.135) (end 130.75 59.15) (width 1) (layer "B.Cu") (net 6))
 (segment (start 158.3 84.7) (end 155 88) (width 1) (layer "F.Cu") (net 37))
 (segment (start 155 88) (end 155 99) (width 1) (layer "F.Cu") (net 37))
 (segment (start 126.3 136.85) (end 141.1 136.85) (width 1) (layer "F.Cu") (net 37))
 (segment (start 119 99) (end 119 129.55) (width 1) (layer "F.Cu") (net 37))
 (segment (start 155 99) (end 119 99) (width 1) (layer "F.Cu") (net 37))
 (segment (start 119 129.55) (end 126.3 136.85) (width 1) (layer "F.Cu") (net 37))
 (segment (start 141.1 136.85) (end 144.25 133.7) (width 1) (layer "F.Cu") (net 37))
 (segment (start 144.25 133.7) (end 144.25 131.05) (width 1) (layer "F.Cu") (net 37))
 (segment (start 144.22 127.4) (end 144.22 131.02) (width 1) (layer "B.Cu") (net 37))
 (segment (start 161.8 84.48) (end 158.52 84.48) (width 1) (layer "B.Cu") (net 37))
 (segment (start 158.52 84.48) (end 158.3 84.7) (width 1) (layer "B.Cu") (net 37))
 (segment (start 144.22 131.02) (end 144.25 131.05) (width 1) (layer "B.Cu") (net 37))
 (segment (start 124.75 83.25) (end 143.3 83.25) (width 1) (layer "B.Cu") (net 19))
 (segment (start 143.25 86.61) (end 143.25 83.3) (width 0.8) (layer "B.Cu") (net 19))
 (segment (start 143.25 83.3) (end 143.3 83.25) (width 0.8) (layer "B.Cu") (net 19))
 (segment (start 122.45 92.05) (end 122.45 85.55) (width 1) (layer "B.Cu") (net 19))
 (segment (start 122.45 85.55) (end 124 84) (width 1) (layer "B.Cu") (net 19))
 (segment (start 124 84) (end 124.75 83.25) (width 1) (layer "B.Cu") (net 19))
 (segment (start 123.81 94.59) (end 124.9 93.5) (width 1) (layer "B.Cu") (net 16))
 (segment (start 124.9 93.5) (end 124.9 92.6) (width 1) (layer "B.Cu") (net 16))
 (segment (start 132.7 91.55) (end 150.41 91.55) (width 1) (layer "B.Cu") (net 16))
 (segment (start 132.7 89.015) (end 132.7 91.55) (width 0.8) (layer "B.Cu") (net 16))
 (segment (start 122.45 94.59) (end 123.81 94.59) (width 1) (layer "B.Cu") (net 16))
 (segment (start 124.9 92.6) (end 125.95 91.55) (width 1) (layer "B.Cu") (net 16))
 (segment (start 150.41 91.55) (end 150.4875 91.6275) (width 1) (layer "B.Cu") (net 16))
 (segment (start 125.95 91.55) (end 132.7 91.55) (width 1) (layer "B.Cu") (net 16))
 (segment (start 127.765 133.64) (end 125.125 131) (width 1) (layer "B.Cu") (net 18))
 (segment (start 120 57) (end 124.405 57) (width 1) (layer "B.Cu") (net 18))
 (segment (start 125.125 131) (end 121 131) (width 1) (layer "B.Cu") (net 18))
 (segment (start 118 98) (end 118 59) (width 1) (layer "B.Cu") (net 18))
 (segment (start 124.405 57) (end 127.765 53.64) (width 1) (layer "B.Cu") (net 18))
 (segment (start 126 101.56) (end 126.44 102) (width 1) (layer "B.Cu") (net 18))
 (segment (start 120.05 130.05) (end 120.05 100.05) (width 1) (layer "B.Cu") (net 18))
 (segment (start 121 131) (end 120.05 130.05) (width 1) (layer "B.Cu") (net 18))
 (segment (start 118 59) (end 120 57) (width 1) (layer "B.Cu") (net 18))
 (segment (start 121 99) (end 126 99) (width 1) (layer "B.Cu") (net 18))
 (segment (start 120 100) (end 121 99) (width 1) (layer "B.Cu") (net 18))
 (segment (start 120 100) (end 118 98) (width 1) (layer "B.Cu") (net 18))
 (segment (start 120.05 100.05) (end 120 100) (width 1) (layer "B.Cu") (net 18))
 (segment (start 126 99) (end 126 101.56) (width 1) (layer "B.Cu") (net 18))
 (segment (start 145.365 89.15) (end 150.4875 84.0275) (width 0.8) (layer "B.Cu") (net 15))
 (segment (start 136.5 86.45) (end 132.725 86.45) (width 0.8) (layer "B.Cu") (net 15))
 (segment (start 132.725 86.45) (end 132.7 86.475) (width 0.8) (layer "B.Cu") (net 15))
 (segment (start 132.725 86.45) (end 132.7 86.475) (width 0.8) (layer "B.Cu") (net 15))
 (segment (start 139.2 89.15) (end 136.5 86.45) (width 0.8) (layer "B.Cu") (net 15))
 (segment (start 143.25 89.15) (end 145.365 89.15) (width 0.8) (layer "B.Cu") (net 15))
 (segment (start 143.25 89.15) (end 139.2 89.15) (width 0.8) (layer "B.Cu") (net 15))
 (segment (start 143.25 89.15) (end 140.15 89.15) (width 0.8) (layer "B.Cu") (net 15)))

